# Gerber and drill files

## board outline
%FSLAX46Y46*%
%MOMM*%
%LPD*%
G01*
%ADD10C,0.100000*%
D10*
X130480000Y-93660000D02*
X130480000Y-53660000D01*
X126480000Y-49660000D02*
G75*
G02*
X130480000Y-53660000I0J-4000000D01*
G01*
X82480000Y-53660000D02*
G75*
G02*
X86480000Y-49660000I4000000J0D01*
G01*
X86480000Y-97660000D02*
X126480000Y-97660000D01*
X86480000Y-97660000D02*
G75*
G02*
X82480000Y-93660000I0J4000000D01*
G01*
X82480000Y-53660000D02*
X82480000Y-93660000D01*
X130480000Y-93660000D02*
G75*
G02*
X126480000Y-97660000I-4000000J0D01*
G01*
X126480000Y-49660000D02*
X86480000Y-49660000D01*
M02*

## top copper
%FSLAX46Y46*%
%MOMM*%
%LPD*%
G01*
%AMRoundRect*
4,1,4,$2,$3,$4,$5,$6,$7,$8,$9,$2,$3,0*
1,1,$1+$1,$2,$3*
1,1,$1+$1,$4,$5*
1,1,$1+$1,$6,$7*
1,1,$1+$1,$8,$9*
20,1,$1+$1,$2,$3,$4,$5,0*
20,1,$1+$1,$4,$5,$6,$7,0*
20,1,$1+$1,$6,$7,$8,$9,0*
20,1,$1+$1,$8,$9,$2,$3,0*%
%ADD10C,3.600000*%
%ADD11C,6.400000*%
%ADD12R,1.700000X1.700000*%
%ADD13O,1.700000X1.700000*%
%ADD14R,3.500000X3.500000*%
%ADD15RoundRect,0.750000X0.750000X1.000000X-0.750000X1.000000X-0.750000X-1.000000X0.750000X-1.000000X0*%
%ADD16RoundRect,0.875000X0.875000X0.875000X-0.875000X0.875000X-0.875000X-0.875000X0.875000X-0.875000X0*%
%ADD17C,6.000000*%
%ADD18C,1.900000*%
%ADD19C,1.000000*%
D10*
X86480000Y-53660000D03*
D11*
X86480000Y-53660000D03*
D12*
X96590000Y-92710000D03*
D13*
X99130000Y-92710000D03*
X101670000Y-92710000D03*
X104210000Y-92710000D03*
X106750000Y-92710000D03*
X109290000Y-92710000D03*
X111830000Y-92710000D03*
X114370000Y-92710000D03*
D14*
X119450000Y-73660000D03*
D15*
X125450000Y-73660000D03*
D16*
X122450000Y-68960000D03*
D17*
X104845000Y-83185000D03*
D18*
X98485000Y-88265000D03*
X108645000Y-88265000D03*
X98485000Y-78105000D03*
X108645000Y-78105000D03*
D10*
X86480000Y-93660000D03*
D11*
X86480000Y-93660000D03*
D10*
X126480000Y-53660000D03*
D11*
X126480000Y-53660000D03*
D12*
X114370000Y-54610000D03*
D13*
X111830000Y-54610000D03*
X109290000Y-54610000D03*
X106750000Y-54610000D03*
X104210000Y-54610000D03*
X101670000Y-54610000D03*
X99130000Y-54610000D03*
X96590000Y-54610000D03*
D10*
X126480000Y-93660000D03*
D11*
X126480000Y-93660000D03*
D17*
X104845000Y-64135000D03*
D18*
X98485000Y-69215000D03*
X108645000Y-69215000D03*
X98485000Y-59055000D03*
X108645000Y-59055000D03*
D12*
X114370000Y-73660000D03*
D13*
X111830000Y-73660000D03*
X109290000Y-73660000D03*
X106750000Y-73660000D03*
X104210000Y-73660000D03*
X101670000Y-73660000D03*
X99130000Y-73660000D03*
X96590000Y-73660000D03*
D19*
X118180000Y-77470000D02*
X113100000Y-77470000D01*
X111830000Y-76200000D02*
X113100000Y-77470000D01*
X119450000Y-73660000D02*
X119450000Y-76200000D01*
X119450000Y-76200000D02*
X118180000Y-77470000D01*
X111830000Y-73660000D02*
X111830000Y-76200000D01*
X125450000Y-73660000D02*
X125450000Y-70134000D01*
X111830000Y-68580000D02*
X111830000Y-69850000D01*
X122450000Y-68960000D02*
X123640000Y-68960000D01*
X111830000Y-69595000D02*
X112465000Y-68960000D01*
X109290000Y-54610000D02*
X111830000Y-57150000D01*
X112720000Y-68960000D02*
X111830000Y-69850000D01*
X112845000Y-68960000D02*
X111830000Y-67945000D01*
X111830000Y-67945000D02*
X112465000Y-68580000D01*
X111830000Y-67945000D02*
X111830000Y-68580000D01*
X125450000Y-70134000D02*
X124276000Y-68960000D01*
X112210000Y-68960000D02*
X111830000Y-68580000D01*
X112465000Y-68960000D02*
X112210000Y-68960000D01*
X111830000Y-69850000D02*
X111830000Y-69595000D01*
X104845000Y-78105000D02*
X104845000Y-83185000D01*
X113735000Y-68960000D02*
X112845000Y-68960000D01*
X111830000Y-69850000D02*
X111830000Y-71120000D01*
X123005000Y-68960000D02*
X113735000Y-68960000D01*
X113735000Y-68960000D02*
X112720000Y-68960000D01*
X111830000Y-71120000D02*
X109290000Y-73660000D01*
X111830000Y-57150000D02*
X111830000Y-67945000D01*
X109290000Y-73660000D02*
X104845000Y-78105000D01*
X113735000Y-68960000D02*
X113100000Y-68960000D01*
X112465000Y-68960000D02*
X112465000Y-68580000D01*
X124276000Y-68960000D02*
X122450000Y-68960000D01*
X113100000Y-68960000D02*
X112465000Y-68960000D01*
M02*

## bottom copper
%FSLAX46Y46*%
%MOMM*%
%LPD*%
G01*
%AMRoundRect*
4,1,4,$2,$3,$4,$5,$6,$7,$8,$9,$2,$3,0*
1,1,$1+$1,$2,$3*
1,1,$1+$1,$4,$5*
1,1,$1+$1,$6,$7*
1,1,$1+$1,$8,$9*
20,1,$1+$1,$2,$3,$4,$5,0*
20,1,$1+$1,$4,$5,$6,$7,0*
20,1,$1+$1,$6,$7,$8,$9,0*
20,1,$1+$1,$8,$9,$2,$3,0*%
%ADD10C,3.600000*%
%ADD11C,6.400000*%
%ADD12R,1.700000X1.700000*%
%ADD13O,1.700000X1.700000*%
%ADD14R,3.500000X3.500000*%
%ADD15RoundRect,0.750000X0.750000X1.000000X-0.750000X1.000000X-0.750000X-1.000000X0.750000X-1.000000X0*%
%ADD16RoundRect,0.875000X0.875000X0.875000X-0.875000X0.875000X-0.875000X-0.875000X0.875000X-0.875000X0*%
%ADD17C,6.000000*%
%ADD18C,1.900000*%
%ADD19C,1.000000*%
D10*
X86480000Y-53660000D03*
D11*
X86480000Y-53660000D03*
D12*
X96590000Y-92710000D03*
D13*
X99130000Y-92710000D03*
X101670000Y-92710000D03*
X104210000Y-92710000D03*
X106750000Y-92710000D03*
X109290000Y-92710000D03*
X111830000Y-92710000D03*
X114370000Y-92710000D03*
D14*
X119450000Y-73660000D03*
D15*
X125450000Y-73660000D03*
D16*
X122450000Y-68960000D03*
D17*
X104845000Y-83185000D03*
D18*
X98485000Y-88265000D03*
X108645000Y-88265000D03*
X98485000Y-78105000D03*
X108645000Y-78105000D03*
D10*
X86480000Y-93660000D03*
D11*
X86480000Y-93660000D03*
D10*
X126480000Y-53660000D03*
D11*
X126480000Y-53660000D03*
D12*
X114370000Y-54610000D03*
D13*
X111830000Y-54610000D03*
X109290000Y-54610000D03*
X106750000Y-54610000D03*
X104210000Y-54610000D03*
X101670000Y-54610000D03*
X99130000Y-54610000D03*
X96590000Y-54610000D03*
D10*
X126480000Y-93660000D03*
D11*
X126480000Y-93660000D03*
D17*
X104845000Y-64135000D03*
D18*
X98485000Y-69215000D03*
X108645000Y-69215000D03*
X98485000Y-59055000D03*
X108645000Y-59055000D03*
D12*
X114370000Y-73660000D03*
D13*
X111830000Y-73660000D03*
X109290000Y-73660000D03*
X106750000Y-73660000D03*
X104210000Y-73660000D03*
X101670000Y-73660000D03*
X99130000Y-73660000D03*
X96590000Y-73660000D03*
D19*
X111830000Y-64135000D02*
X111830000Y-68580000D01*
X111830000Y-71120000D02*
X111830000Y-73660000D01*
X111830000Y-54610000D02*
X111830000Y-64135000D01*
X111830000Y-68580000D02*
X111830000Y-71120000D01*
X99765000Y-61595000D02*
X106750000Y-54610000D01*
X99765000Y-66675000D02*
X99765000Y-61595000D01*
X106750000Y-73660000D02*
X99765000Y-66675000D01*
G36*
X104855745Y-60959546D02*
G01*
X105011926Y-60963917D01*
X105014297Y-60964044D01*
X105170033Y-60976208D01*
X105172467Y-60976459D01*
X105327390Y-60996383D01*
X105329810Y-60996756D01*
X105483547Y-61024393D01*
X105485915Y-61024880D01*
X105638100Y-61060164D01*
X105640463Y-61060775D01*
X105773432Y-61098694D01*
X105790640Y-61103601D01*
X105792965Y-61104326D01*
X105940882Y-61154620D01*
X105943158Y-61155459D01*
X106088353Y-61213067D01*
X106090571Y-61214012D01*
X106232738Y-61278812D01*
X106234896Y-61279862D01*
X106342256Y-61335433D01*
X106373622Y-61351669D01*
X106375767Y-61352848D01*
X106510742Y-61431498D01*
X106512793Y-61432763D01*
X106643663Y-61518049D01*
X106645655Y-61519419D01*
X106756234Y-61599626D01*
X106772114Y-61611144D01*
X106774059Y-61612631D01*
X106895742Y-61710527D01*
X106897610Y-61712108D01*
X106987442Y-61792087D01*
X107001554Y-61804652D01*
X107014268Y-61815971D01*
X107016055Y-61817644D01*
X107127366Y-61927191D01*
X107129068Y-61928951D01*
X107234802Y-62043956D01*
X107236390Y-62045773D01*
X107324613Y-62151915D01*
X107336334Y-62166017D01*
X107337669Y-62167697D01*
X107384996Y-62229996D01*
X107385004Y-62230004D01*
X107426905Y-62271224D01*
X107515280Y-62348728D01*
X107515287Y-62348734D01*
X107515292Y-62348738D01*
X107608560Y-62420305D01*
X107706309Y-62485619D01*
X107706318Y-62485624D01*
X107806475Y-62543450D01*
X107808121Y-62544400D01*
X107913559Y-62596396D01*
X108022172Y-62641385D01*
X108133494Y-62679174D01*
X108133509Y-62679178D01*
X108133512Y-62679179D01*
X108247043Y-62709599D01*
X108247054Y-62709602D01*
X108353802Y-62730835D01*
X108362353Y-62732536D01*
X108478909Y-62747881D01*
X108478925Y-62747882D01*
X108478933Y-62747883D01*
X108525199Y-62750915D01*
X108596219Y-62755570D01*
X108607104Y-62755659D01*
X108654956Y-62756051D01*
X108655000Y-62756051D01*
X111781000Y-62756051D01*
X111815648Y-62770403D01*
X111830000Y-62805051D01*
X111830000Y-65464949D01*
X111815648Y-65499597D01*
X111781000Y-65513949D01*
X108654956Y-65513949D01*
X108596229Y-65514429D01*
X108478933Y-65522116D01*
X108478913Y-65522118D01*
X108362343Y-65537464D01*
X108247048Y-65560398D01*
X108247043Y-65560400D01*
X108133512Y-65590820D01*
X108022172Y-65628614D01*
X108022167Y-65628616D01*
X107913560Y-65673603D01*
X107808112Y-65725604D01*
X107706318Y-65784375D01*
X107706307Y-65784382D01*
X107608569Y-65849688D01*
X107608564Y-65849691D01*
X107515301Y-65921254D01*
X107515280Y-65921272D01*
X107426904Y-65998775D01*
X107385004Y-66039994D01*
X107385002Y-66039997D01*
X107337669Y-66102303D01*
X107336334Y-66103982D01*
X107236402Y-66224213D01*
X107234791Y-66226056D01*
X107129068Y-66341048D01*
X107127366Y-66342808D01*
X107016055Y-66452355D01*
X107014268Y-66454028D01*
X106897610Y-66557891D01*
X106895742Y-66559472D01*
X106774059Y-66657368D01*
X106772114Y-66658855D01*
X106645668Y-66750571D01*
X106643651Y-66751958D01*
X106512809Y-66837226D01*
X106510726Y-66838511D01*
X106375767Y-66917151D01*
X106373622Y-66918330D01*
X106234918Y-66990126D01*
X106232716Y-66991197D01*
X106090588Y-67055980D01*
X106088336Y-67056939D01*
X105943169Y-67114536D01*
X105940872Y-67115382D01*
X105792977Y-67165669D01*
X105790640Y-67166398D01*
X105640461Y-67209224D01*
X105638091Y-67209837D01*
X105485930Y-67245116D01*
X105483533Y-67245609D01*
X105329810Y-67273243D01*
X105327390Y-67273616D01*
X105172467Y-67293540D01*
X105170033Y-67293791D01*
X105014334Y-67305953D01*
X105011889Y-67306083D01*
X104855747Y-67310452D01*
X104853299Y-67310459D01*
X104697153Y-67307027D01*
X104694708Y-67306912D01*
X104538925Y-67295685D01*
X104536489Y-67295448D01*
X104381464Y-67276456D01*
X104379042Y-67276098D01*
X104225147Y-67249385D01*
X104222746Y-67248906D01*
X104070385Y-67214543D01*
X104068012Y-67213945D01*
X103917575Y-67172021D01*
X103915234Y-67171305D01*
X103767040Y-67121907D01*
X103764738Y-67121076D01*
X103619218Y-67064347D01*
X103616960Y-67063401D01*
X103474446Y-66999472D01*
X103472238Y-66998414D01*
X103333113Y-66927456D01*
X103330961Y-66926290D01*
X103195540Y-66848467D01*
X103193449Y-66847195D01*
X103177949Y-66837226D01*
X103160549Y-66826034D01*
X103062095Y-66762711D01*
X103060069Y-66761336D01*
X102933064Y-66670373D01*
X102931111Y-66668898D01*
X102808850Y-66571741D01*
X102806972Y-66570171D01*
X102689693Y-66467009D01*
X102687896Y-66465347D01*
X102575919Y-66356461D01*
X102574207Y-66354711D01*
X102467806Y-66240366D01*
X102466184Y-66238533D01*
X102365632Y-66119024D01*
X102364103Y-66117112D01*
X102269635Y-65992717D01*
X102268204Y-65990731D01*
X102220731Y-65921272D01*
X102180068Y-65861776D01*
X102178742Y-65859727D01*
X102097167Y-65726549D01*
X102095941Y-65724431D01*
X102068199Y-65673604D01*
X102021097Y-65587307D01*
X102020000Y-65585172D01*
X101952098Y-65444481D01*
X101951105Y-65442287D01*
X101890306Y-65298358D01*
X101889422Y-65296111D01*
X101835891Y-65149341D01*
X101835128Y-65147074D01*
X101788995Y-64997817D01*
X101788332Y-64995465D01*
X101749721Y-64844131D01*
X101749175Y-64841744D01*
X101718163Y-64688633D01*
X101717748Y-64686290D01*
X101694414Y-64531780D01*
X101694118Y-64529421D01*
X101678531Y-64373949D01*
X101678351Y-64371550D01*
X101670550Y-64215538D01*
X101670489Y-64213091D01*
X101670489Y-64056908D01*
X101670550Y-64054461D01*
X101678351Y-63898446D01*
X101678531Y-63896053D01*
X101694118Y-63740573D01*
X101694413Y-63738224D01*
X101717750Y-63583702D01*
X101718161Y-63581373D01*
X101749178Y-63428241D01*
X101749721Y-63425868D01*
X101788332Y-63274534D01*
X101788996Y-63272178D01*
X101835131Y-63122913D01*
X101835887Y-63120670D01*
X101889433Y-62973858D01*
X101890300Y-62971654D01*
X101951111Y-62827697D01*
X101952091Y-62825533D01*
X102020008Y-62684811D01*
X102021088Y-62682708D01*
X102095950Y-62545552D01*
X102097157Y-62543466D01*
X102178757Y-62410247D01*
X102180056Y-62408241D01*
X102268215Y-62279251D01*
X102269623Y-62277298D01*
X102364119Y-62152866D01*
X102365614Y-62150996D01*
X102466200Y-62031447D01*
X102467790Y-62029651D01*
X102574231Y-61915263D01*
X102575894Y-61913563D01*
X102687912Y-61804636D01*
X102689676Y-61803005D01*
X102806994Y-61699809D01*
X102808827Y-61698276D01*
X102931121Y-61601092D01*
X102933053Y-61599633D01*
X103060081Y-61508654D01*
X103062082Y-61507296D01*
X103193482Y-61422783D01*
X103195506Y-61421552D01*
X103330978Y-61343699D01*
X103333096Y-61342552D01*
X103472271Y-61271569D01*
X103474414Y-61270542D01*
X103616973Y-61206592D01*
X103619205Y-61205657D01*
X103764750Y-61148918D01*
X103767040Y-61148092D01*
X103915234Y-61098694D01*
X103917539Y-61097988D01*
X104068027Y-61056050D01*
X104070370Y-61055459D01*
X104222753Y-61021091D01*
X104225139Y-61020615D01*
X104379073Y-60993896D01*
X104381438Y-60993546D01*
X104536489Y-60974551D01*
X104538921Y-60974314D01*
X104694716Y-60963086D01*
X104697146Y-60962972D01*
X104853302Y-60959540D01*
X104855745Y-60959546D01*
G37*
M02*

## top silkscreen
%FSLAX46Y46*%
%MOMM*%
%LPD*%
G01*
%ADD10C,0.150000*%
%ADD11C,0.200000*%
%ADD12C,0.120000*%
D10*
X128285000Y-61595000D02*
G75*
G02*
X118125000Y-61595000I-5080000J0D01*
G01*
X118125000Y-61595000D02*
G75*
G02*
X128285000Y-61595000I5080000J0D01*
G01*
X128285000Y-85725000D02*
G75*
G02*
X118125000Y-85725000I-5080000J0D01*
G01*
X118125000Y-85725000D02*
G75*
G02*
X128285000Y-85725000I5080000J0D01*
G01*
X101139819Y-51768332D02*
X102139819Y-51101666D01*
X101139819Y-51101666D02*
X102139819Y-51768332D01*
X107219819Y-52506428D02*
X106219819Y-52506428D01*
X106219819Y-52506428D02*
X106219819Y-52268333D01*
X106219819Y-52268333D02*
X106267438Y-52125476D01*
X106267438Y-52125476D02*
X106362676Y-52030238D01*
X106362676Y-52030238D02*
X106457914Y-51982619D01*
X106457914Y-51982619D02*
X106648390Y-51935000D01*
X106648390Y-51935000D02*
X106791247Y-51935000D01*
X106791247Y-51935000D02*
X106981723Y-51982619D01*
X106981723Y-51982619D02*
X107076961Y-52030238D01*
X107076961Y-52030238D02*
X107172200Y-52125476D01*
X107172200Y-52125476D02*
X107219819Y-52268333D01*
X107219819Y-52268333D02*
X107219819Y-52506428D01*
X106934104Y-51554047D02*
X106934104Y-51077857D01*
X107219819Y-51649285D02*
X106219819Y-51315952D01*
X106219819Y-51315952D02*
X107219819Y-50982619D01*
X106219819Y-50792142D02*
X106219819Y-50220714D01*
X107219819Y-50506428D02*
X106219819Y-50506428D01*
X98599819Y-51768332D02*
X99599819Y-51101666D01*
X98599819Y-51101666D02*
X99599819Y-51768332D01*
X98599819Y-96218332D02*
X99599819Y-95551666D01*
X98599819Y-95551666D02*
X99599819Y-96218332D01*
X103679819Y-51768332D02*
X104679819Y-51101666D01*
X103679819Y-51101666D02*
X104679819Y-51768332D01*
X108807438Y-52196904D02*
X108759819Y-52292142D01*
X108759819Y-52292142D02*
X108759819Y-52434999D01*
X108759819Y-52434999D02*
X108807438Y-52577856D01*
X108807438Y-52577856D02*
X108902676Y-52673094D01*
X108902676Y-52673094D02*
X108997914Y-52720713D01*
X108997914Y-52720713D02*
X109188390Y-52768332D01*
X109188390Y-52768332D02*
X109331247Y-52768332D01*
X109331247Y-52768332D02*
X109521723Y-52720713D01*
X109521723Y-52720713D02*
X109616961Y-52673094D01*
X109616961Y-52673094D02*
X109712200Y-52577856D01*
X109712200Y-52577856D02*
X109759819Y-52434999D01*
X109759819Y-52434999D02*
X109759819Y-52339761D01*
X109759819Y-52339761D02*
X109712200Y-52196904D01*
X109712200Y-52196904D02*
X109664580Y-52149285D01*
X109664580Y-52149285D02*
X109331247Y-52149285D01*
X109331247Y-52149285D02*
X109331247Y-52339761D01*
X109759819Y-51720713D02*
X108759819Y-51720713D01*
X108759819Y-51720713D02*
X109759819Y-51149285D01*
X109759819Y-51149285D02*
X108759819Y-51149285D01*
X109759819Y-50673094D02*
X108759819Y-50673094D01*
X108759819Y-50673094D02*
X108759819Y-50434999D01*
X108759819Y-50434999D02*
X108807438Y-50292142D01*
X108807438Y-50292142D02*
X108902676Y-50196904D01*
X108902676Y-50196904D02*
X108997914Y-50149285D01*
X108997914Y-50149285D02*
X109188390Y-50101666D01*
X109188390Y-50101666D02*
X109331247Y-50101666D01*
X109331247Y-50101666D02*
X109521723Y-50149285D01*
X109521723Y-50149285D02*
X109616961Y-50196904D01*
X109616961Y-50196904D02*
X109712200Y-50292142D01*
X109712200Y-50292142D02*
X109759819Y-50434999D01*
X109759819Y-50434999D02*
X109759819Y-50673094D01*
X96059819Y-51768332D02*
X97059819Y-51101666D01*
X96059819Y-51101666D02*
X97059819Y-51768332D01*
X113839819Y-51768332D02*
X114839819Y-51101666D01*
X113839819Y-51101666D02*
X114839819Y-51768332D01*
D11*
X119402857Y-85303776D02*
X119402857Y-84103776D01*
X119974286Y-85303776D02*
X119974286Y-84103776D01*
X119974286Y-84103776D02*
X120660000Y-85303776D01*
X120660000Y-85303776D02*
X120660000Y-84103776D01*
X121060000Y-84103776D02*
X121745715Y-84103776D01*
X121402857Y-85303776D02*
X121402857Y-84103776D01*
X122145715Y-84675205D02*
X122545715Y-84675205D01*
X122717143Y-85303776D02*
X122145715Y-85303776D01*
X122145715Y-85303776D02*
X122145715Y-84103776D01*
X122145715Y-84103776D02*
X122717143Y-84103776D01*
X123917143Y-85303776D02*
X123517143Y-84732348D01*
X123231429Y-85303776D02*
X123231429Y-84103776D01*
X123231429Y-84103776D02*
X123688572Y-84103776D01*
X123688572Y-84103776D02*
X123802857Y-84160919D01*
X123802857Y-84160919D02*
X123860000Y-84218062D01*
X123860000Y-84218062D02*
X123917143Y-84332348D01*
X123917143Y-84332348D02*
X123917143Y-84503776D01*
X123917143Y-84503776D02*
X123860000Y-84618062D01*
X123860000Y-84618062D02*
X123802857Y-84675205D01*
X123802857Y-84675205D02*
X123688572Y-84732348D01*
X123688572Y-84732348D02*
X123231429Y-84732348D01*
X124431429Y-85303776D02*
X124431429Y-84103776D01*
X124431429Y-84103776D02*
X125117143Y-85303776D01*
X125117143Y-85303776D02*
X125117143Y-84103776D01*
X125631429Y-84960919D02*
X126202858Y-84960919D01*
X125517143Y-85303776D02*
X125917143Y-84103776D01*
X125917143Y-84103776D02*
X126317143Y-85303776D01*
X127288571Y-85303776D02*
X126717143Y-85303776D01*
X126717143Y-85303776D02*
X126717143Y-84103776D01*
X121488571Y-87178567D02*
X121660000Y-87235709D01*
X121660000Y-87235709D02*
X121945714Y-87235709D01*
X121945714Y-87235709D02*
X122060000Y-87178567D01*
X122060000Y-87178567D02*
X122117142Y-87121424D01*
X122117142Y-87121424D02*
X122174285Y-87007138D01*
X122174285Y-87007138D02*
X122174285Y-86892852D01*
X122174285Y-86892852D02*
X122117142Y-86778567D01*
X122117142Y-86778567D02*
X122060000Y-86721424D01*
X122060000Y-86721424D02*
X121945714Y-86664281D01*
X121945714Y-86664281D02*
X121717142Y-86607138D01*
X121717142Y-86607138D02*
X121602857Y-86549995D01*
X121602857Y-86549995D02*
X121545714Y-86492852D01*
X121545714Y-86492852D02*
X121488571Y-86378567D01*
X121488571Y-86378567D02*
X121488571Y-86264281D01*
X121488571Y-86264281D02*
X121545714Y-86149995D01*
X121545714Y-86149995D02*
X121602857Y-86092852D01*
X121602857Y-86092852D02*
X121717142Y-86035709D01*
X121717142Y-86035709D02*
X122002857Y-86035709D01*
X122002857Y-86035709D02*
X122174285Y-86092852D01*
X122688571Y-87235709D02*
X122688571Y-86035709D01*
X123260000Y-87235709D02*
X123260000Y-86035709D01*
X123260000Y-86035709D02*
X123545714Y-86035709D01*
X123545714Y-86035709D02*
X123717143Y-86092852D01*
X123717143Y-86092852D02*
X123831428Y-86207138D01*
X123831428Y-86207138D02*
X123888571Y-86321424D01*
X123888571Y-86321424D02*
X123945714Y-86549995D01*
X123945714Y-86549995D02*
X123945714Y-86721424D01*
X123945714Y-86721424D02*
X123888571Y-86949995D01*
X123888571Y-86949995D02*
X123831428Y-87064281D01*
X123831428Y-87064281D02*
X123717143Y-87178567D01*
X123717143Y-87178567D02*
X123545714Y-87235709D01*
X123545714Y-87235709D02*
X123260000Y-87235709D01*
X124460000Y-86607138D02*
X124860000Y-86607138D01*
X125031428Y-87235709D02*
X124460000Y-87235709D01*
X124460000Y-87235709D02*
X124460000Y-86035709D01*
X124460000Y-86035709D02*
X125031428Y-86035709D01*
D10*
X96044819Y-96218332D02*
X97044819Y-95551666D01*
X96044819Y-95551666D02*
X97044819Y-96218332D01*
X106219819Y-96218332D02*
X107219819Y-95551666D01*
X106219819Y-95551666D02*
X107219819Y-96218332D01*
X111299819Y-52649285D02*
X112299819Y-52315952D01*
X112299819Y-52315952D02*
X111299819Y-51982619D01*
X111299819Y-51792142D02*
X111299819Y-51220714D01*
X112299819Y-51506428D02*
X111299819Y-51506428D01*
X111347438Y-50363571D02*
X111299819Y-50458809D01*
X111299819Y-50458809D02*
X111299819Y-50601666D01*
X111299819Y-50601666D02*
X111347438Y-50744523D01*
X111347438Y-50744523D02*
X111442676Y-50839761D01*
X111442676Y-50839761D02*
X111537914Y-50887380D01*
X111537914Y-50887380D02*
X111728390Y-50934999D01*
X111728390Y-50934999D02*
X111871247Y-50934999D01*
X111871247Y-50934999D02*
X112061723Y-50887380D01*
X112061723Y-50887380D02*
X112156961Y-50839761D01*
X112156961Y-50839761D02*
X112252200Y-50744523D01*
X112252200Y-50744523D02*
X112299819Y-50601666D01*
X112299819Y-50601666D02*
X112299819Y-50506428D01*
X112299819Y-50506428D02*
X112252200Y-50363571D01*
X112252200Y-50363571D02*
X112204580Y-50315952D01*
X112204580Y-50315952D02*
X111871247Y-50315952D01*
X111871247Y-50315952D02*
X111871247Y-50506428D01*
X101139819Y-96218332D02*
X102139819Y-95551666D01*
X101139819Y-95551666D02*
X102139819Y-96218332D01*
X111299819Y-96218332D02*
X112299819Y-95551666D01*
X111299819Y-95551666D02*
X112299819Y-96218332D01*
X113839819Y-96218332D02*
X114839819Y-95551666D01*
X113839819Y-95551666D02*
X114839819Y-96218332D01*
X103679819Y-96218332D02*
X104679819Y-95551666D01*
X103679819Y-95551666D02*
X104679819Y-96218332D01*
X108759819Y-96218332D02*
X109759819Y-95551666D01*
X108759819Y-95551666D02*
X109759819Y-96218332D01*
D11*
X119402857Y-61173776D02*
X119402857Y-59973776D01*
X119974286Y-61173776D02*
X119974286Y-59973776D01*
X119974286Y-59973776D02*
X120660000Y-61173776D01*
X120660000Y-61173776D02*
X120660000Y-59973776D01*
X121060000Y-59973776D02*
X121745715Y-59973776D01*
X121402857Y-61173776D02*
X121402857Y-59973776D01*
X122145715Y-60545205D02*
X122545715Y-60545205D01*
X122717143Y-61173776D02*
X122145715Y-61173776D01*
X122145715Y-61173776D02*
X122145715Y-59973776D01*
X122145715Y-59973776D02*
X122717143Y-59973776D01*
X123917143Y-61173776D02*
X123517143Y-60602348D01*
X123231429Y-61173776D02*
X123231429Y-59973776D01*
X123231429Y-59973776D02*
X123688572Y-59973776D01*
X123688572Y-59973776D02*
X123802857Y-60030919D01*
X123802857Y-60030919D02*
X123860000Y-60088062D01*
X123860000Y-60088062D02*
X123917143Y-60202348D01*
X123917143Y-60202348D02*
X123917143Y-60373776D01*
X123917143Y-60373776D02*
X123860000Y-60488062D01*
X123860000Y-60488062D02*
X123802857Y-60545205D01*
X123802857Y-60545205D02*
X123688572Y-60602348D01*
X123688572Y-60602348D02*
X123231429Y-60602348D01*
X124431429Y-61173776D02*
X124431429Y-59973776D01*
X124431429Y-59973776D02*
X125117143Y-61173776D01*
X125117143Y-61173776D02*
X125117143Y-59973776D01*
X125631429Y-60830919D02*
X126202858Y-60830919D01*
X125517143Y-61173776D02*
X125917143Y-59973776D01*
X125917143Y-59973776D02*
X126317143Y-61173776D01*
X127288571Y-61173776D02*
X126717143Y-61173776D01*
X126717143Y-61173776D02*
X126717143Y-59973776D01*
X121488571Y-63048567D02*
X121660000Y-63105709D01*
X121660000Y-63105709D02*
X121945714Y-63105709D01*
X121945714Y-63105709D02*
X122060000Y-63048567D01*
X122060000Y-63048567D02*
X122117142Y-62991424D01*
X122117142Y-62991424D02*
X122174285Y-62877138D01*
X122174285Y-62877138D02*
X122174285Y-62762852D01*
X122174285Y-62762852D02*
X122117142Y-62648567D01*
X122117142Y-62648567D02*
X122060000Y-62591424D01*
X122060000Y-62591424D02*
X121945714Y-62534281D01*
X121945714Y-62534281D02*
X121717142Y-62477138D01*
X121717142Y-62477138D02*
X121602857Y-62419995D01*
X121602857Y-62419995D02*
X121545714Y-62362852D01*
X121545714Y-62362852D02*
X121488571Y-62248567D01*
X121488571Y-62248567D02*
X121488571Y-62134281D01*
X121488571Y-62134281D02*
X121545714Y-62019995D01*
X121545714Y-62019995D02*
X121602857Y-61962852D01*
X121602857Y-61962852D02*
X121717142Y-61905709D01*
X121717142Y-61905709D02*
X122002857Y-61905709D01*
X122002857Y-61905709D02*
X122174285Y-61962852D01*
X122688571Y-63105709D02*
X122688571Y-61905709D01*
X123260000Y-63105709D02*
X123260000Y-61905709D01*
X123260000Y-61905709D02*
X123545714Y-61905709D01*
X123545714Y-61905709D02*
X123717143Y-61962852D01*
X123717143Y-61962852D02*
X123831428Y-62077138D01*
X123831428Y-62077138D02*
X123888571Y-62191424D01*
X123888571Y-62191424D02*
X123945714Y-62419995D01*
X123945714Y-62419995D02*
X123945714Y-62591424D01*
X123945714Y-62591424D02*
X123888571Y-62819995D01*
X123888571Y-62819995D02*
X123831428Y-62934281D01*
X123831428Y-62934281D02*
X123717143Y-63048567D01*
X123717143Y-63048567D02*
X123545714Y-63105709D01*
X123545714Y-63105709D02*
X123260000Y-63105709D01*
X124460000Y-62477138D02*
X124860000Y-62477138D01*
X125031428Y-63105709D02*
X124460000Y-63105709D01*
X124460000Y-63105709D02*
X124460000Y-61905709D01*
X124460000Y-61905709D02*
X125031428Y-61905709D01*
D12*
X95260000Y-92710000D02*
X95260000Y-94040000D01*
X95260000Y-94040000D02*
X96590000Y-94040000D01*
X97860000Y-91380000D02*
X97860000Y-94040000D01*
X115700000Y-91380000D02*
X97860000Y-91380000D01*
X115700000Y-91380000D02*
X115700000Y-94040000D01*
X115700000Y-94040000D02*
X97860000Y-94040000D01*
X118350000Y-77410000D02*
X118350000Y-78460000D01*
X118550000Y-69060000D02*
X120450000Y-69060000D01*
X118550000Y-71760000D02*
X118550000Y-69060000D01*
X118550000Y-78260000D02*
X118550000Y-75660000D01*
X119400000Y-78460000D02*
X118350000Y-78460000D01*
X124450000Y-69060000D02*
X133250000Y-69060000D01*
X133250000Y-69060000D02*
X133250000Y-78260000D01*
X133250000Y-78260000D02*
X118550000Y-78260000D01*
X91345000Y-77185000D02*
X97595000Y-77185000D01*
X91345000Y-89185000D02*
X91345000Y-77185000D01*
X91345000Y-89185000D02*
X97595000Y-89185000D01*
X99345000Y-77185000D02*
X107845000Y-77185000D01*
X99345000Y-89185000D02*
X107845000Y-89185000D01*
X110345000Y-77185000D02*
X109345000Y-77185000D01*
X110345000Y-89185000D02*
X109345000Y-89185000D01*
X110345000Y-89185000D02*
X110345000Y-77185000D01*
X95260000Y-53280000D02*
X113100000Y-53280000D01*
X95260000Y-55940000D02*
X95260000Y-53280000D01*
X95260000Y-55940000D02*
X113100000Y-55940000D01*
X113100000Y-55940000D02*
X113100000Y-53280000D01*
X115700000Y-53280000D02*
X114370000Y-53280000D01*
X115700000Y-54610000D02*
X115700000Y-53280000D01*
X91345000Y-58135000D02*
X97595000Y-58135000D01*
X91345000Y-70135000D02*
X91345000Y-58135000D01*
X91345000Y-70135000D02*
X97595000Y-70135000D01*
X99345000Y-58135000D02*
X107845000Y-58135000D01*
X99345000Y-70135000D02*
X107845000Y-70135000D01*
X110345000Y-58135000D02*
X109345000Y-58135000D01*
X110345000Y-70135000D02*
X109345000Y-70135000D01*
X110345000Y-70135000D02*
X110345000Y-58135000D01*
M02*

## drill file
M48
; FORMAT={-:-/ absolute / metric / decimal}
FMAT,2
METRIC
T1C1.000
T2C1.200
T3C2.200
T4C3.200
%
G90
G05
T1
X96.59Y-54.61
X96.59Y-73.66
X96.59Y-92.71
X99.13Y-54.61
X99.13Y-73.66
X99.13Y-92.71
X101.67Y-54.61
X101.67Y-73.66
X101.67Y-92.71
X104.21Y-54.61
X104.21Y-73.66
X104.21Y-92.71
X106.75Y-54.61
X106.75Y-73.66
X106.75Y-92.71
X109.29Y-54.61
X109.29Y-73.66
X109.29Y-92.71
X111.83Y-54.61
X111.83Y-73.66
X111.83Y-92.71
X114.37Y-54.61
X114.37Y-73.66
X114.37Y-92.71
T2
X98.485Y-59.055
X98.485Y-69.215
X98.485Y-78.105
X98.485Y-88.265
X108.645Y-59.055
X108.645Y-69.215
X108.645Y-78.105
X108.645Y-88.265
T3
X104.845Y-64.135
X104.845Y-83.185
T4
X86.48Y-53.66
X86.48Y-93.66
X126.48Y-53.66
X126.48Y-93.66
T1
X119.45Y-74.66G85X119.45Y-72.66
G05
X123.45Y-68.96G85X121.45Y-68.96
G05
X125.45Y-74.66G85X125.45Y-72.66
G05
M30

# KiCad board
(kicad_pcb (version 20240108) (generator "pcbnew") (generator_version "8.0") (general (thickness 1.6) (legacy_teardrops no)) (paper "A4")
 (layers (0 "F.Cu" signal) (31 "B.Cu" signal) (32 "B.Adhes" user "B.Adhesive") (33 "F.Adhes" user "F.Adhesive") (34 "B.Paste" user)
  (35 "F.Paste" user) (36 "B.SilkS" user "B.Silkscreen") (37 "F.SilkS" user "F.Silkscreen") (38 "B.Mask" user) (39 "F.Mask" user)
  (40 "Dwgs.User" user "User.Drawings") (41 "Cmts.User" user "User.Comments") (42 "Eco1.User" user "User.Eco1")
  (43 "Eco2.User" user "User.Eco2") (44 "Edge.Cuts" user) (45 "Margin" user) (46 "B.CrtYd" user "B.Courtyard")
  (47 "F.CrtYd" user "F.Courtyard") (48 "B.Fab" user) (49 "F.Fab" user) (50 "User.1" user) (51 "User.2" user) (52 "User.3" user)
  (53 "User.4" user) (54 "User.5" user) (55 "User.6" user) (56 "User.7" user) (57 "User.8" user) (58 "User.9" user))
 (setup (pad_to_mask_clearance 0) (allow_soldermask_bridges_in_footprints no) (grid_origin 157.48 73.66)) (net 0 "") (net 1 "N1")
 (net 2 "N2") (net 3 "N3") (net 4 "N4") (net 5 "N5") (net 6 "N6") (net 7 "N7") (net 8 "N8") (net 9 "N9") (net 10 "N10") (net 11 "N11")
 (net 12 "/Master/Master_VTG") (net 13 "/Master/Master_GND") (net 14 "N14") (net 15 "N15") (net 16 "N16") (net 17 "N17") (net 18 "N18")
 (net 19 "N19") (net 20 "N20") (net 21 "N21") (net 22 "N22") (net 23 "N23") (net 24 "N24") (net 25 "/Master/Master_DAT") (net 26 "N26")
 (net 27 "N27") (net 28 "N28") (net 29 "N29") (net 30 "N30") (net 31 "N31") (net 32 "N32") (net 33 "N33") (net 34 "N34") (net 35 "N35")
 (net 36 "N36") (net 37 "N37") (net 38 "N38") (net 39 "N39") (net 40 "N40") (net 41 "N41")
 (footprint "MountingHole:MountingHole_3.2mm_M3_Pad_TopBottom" (layer "F.Cu") (at 86.48 53.66)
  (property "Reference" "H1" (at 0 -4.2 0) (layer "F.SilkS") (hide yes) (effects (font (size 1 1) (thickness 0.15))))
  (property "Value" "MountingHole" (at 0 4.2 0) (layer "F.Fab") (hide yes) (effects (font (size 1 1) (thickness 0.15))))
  (pad "1" thru_hole circle (at 0 0) (size 3.6 3.6) (drill 3.2) (layers "*.Cu" "*.Mask") (remove_unused_layers no) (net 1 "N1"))
  (pad "1" connect circle (at 0 0) (size 6.4 6.4) (layers "F.Cu" "F.Mask") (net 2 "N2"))
  (pad "1" connect circle (at 0 0) (size 6.4 6.4) (layers "B.Cu" "B.Mask") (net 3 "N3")))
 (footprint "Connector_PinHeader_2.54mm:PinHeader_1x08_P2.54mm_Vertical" (layer "F.Cu") (at 96.59 92.71 90)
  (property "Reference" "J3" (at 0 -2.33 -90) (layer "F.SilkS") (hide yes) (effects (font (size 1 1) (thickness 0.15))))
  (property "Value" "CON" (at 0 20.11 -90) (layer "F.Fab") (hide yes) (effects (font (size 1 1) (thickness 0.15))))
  (fp_line (start 0 -1.33) (end -1.33 -1.33) (stroke (width 0.12) (type solid)) (layer "F.SilkS"))
  (fp_line (start -1.33 -1.33) (end -1.33 0) (stroke (width 0.12) (type solid)) (layer "F.SilkS"))
  (fp_line (start 1.33 1.27) (end -1.33 1.27) (stroke (width 0.12) (type solid)) (layer "F.SilkS"))
  (fp_line (start 1.33 19.11) (end 1.33 1.27) (stroke (width 0.12) (type solid)) (layer "F.SilkS"))
  (fp_line (start 1.33 19.11) (end -1.33 19.11) (stroke (width 0.12) (type solid)) (layer "F.SilkS"))
  (fp_line (start -1.33 19.11) (end -1.33 1.27) (stroke (width 0.12) (type solid)) (layer "F.SilkS"))
  (pad "1" thru_hole rect (at 0 0 90) (size 1.7 1.7) (drill 1) (layers "*.Cu" "*.Mask") (remove_unused_layers no) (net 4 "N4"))
  (pad "2" thru_hole oval (at 0 2.54 90) (size 1.7 1.7) (drill 1) (layers "*.Cu" "*.Mask") (remove_unused_layers no) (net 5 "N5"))
  (pad "3" thru_hole oval (at 0 5.08 90) (size 1.7 1.7) (drill 1) (layers "*.Cu" "*.Mask") (remove_unused_layers no) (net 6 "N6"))
  (pad "4" thru_hole oval (at 0 7.62 90) (size 1.7 1.7) (drill 1) (layers "*.Cu" "*.Mask") (remove_unused_layers no) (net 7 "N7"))
  (pad "5" thru_hole oval (at 0 10.16 90) (size 1.7 1.7) (drill 1) (layers "*.Cu" "*.Mask") (remove_unused_layers no) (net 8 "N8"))
  (pad "6" thru_hole oval (at 0 12.7 90) (size 1.7 1.7) (drill 1) (layers "*.Cu" "*.Mask") (remove_unused_layers no) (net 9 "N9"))
  (pad "7" thru_hole oval (at 0 15.24 90) (size 1.7 1.7) (drill 1) (layers "*.Cu" "*.Mask") (remove_unused_layers no) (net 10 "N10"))
  (pad "8" thru_hole oval (at 0 17.78 90) (size 1.7 1.7) (drill 1) (layers "*.Cu" "*.Mask") (remove_unused_layers no) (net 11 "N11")))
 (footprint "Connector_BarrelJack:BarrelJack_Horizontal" (layer "F.Cu") (at 119.45 73.66 180)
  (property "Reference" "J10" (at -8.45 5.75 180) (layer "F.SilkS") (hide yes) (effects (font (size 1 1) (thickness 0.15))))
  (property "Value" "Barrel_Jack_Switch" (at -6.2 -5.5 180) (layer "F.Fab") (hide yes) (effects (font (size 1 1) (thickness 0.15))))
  (fp_line (start 1.1 -3.75) (end 1.1 -4.8) (stroke (width 0.12) (type solid)) (layer "F.SilkS"))
  (fp_line (start 0.9 4.6) (end -1 4.6) (stroke (width 0.12) (type solid)) (layer "F.SilkS"))
  (fp_line (start 0.9 1.9) (end 0.9 4.6) (stroke (width 0.12) (type solid)) (layer "F.SilkS"))
  (fp_line (start 0.9 -4.6) (end 0.9 -2) (stroke (width 0.12) (type solid)) (layer "F.SilkS"))
  (fp_line (start 0.05 -4.8) (end 1.1 -4.8) (stroke (width 0.12) (type solid)) (layer "F.SilkS"))
  (fp_line (start -5 4.6) (end -13.8 4.6) (stroke (width 0.12) (type solid)) (layer "F.SilkS"))
  (fp_line (start -13.8 4.6) (end -13.8 -4.6) (stroke (width 0.12) (type solid)) (layer "F.SilkS"))
  (fp_line (start -13.8 -4.6) (end 0.9 -4.6) (stroke (width 0.12) (type solid)) (layer "F.SilkS"))
  (pad "1" thru_hole rect (at 0 0 180) (size 3.5 3.5) (drill oval 1 3) (layers "*.Cu" "*.Mask") (remove_unused_layers no)
   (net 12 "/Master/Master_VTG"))
  (pad "2" thru_hole roundrect (at -6 0 180) (size 3 3.5) (drill oval 1 3) (layers "*.Cu" "*.Mask") (remove_unused_layers no)
   (roundrect_rratio 0.25) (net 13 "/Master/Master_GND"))
  (pad "3" thru_hole roundrect (at -3 4.7 180) (size 3.5 3.5) (drill oval 3 1) (layers "*.Cu" "*.Mask") (remove_unused_layers no)
   (roundrect_rratio 0.25) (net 13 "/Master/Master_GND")))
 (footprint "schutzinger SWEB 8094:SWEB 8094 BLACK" (layer "F.Cu") (at 104.845 83.185 90)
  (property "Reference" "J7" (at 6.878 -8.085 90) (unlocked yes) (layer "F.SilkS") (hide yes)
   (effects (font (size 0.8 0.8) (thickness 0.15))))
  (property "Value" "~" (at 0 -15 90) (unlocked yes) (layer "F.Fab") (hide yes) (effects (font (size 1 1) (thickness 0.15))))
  (fp_line (start 6 -13.5) (end 6 -7.25) (stroke (width 0.12) (type solid)) (layer "F.SilkS"))
  (fp_line (start -6 -13.5) (end 6 -13.5) (stroke (width 0.12) (type solid)) (layer "F.SilkS"))
  (fp_line (start -6 -13.5) (end -6 -7.25) (stroke (width 0.12) (type solid)) (layer "F.SilkS"))
  (fp_line (start 6 -5.5) (end 6 3) (stroke (width 0.12) (type solid)) (layer "F.SilkS"))
  (fp_line (start -6 -5.5) (end -6 3) (stroke (width 0.12) (type solid)) (layer "F.SilkS"))
  (fp_line (start 6 5.5) (end 6 4.5) (stroke (width 0.12) (type solid)) (layer "F.SilkS"))
  (fp_line (start -6 5.5) (end -6 4.5) (stroke (width 0.12) (type solid)) (layer "F.SilkS"))
  (fp_line (start -6 5.5) (end 6 5.5) (stroke (width 0.12) (type solid)) (layer "F.SilkS"))
  (pad "1" thru_hole circle (at 0 0 90) (size 6 6) (drill 2.2) (layers "*.Cu" "*.Mask") (remove_unused_layers no)
   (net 13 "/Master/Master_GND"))
  (pad "MP" thru_hole circle (at -5.08 -6.36 90) (size 1.9 1.9) (drill 1.2) (layers "*.Cu" "*.Mask") (remove_unused_layers no)
   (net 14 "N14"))
  (pad "MP" thru_hole circle (at -5.08 3.8 90) (size 1.9 1.9) (drill 1.2) (layers "*.Cu" "*.Mask") (remove_unused_layers no) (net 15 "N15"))
  (pad "MP" thru_hole circle (at 5.08 -6.36 90) (size 1.9 1.9) (drill 1.2) (layers "*.Cu" "*.Mask") (remove_unused_layers no) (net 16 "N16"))
  (pad "MP" thru_hole circle (at 5.08 3.8 90) (size 1.9 1.9) (drill 1.2) (layers "*.Cu" "*.Mask") (remove_unused_layers no) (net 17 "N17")))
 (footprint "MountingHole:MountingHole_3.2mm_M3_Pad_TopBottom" (layer "F.Cu") (at 86.48 93.66)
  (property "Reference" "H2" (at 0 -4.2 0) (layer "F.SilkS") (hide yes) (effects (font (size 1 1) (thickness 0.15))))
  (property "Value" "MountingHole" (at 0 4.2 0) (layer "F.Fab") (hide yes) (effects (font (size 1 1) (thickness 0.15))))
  (pad "1" thru_hole circle (at 0 0) (size 3.6 3.6) (drill 3.2) (layers "*.Cu" "*.Mask") (remove_unused_layers no) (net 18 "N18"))
  (pad "1" connect circle (at 0 0) (size 6.4 6.4) (layers "F.Cu" "F.Mask") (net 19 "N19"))
  (pad "1" connect circle (at 0 0) (size 6.4 6.4) (layers "B.Cu" "B.Mask") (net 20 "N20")))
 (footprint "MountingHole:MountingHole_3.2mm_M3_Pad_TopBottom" (layer "F.Cu") (at 126.48 53.66)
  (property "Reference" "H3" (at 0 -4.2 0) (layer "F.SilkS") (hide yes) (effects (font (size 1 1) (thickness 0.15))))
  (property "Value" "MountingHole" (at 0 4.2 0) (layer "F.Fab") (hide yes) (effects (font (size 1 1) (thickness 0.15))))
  (pad "1" thru_hole circle (at 0 0) (size 3.6 3.6) (drill 3.2) (layers "*.Cu" "*.Mask") (remove_unused_layers no) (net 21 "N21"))
  (pad "1" connect circle (at 0 0) (size 6.4 6.4) (layers "F.Cu" "F.Mask") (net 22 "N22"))
  (pad "1" connect circle (at 0 0) (size 6.4 6.4) (layers "B.Cu" "B.Mask") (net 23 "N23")))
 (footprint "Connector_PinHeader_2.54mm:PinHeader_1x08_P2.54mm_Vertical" (layer "F.Cu") (at 114.37 54.61 -90)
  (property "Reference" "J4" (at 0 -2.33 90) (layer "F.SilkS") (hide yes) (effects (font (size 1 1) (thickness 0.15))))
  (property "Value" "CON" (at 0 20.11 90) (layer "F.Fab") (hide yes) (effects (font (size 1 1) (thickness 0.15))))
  (fp_line (start -1.33 19.11) (end -1.33 1.27) (stroke (width 0.12) (type solid)) (layer "F.SilkS"))
  (fp_line (start 1.33 19.11) (end -1.33 19.11) (stroke (width 0.12) (type solid)) (layer "F.SilkS"))
  (fp_line (start 1.33 19.11) (end 1.33 1.27) (stroke (width 0.12) (type solid)) (layer "F.SilkS"))
  (fp_line (start 1.33 1.27) (end -1.33 1.27) (stroke (width 0.12) (type solid)) (layer "F.SilkS"))
  (fp_line (start -1.33 -1.33) (end -1.33 0) (stroke (width 0.12) (type solid)) (layer "F.SilkS"))
  (fp_line (start 0 -1.33) (end -1.33 -1.33) (stroke (width 0.12) (type solid)) (layer "F.SilkS"))
  (pad "1" thru_hole rect (at 0 0 270) (size 1.7 1.7) (drill 1) (layers "*.Cu" "*.Mask") (remove_unused_layers no) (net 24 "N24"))
  (pad "2" thru_hole oval (at 0 2.54 270) (size 1.7 1.7) (drill 1) (layers "*.Cu" "*.Mask") (remove_unused_layers no)
   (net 12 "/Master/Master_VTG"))
  (pad "3" thru_hole oval (at 0 5.08 270) (size 1.7 1.7) (drill 1) (layers "*.Cu" "*.Mask") (remove_unused_layers no)
   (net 13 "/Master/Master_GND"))
  (pad "4" thru_hole oval (at 0 7.62 270) (size 1.7 1.7) (drill 1) (layers "*.Cu" "*.Mask") (remove_unused_layers no)
   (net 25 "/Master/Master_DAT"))
  (pad "5" thru_hole oval (at 0 10.16 270) (size 1.7 1.7) (drill 1) (layers "*.Cu" "*.Mask") (remove_unused_layers no) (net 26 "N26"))
  (pad "6" thru_hole oval (at 0 12.7 270) (size 1.7 1.7) (drill 1) (layers "*.Cu" "*.Mask") (remove_unused_layers no) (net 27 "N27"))
  (pad "7" thru_hole oval (at 0 15.24 270) (size 1.7 1.7) (drill 1) (layers "*.Cu" "*.Mask") (remove_unused_layers no) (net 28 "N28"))
  (pad "8" thru_hole oval (at 0 17.78 270) (size 1.7 1.7) (drill 1) (layers "*.Cu" "*.Mask") (remove_unused_layers no) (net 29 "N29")))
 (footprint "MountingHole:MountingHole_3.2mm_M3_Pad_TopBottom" (layer "F.Cu") (at 126.48 93.66)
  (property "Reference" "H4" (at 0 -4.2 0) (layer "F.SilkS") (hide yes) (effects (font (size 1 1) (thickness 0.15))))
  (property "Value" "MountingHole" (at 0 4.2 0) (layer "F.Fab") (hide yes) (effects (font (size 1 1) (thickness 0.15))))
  (pad "1" thru_hole circle (at 0 0) (size 3.6 3.6) (drill 3.2) (layers "*.Cu" "*.Mask") (remove_unused_layers no) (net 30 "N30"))
  (pad "1" connect circle (at 0 0) (size 6.4 6.4) (layers "F.Cu" "F.Mask") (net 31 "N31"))
  (pad "1" connect circle (at 0 0) (size 6.4 6.4) (layers "B.Cu" "B.Mask") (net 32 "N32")))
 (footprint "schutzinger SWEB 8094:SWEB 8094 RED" (layer "F.Cu") (at 104.845 64.135 90)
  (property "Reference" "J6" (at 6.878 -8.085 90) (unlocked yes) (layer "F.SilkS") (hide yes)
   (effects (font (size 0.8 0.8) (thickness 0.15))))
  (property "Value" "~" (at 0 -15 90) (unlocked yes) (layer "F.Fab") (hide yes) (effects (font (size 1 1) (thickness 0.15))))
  (fp_line (start 6 -13.5) (end 6 -7.25) (stroke (width 0.12) (type solid)) (layer "F.SilkS"))
  (fp_line (start -6 -13.5) (end 6 -13.5) (stroke (width 0.12) (type solid)) (layer "F.SilkS"))
  (fp_line (start -6 -13.5) (end -6 -7.25) (stroke (width 0.12) (type solid)) (layer "F.SilkS"))
  (fp_line (start 6 -5.5) (end 6 3) (stroke (width 0.12) (type solid)) (layer "F.SilkS"))
  (fp_line (start -6 -5.5) (end -6 3) (stroke (width 0.12) (type solid)) (layer "F.SilkS"))
  (fp_line (start 6 5.5) (end 6 4.5) (stroke (width 0.12) (type solid)) (layer "F.SilkS"))
  (fp_line (start -6 5.5) (end -6 4.5) (stroke (width 0.12) (type solid)) (layer "F.SilkS"))
  (fp_line (start -6 5.5) (end 6 5.5) (stroke (width 0.12) (type solid)) (layer "F.SilkS"))
  (pad "1" thru_hole circle (at 0 0 90) (size 6 6) (drill 2.2) (layers "*.Cu" "*.Mask") (remove_unused_layers no)
   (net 12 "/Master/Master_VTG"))
  (pad "MP" thru_hole circle (at -5.08 -6.36 90) (size 1.9 1.9) (drill 1.2) (layers "*.Cu" "*.Mask") (remove_unused_layers no)
   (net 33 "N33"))
  (pad "MP" thru_hole circle (at -5.08 3.8 90) (size 1.9 1.9) (drill 1.2) (layers "*.Cu" "*.Mask") (remove_unused_layers no) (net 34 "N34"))
  (pad "MP" thru_hole circle (at 5.08 -6.36 90) (size 1.9 1.9) (drill 1.2) (layers "*.Cu" "*.Mask") (remove_unused_layers no) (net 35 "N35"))
  (pad "MP" thru_hole circle (at 5.08 3.8 90) (size 1.9 1.9) (drill 1.2) (layers "*.Cu" "*.Mask") (remove_unused_layers no) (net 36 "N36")))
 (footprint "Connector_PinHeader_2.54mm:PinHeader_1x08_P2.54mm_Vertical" (layer "B.Cu") (at 114.37 73.66 90)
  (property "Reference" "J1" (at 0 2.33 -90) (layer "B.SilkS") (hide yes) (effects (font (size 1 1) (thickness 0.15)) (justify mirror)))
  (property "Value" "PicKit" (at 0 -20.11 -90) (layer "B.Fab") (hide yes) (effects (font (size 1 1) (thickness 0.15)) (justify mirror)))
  (pad "1" thru_hole rect (at 0 0 90) (size 1.7 1.7) (drill 1) (layers "*.Cu" "*.Mask") (remove_unused_layers no) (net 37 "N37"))
  (pad "2" thru_hole oval (at 0 -2.54 90) (size 1.7 1.7) (drill 1) (layers "*.Cu" "*.Mask") (remove_unused_layers no)
   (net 12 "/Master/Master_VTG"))
  (pad "3" thru_hole oval (at 0 -5.08 90) (size 1.7 1.7) (drill 1) (layers "*.Cu" "*.Mask") (remove_unused_layers no)
   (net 13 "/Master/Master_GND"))
  (pad "4" thru_hole oval (at 0 -7.62 90) (size 1.7 1.7) (drill 1) (layers "*.Cu" "*.Mask") (remove_unused_layers no)
   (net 25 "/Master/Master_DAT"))
  (pad "5" thru_hole oval (at 0 -10.16 90) (size 1.7 1.7) (drill 1) (layers "*.Cu" "*.Mask") (remove_unused_layers no) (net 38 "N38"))
  (pad "6" thru_hole oval (at 0 -12.7 90) (size 1.7 1.7) (drill 1) (layers "*.Cu" "*.Mask") (remove_unused_layers no) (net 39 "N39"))
  (pad "7" thru_hole oval (at 0 -15.24 90) (size 1.7 1.7) (drill 1) (layers "*.Cu" "*.Mask") (remove_unused_layers no) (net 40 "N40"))
  (pad "8" thru_hole oval (at 0 -17.78 90) (size 1.7 1.7) (drill 1) (layers "*.Cu" "*.Mask") (remove_unused_layers no) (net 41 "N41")))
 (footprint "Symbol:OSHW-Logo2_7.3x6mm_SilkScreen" (layer "B.Cu") (at 86.43 63.5 90)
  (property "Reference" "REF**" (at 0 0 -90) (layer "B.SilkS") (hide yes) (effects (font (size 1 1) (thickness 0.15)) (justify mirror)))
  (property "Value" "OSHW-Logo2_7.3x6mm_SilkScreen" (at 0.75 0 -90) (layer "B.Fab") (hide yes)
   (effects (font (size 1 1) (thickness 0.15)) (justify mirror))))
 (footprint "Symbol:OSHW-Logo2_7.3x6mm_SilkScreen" (layer "B.Cu") (at 86.43 83.82 90)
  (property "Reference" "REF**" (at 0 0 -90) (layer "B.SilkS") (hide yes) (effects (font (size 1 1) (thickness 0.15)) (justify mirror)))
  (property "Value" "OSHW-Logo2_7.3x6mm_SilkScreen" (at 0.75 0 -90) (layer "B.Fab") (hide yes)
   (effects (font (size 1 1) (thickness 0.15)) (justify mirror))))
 (gr_circle (center 123.205 61.595) (end 118.125 61.595) (stroke (width 0.15) (type default)) (fill none) (layer "F.SilkS"))
 (gr_circle (center 123.205 85.725) (end 118.125 85.725) (stroke (width 0.15) (type default)) (fill none) (layer "F.SilkS"))
 (gr_line (start 130.48 93.66) (end 130.48 53.66) (stroke (width 0.1) (type default)) (layer "Edge.Cuts"))
 (gr_arc (start 126.48 49.66) (mid 129.308427 50.831573) (end 130.48 53.66) (stroke (width 0.1) (type default)) (layer "Edge.Cuts"))
 (gr_arc (start 82.48 53.66) (mid 83.651573 50.831573) (end 86.48 49.66) (stroke (width 0.1) (type default)) (layer "Edge.Cuts"))
 (gr_line (start 86.48 97.66) (end 126.48 97.66) (stroke (width 0.1) (type default)) (layer "Edge.Cuts"))
 (gr_arc (start 86.48 97.66) (mid 83.651573 96.488427) (end 82.48 93.66) (stroke (width 0.1) (type default)) (layer "Edge.Cuts"))
 (gr_line (start 82.48 53.66) (end 82.48 93.66) (stroke (width 0.1) (type default)) (layer "Edge.Cuts"))
 (gr_arc (start 130.48 93.66) (mid 129.308427 96.488427) (end 126.48 97.66) (stroke (width 0.1) (type default)) (layer "Edge.Cuts"))
 (gr_line (start 126.48 49.66) (end 86.48 49.66) (stroke (width 0.1) (type default)) (layer "Edge.Cuts"))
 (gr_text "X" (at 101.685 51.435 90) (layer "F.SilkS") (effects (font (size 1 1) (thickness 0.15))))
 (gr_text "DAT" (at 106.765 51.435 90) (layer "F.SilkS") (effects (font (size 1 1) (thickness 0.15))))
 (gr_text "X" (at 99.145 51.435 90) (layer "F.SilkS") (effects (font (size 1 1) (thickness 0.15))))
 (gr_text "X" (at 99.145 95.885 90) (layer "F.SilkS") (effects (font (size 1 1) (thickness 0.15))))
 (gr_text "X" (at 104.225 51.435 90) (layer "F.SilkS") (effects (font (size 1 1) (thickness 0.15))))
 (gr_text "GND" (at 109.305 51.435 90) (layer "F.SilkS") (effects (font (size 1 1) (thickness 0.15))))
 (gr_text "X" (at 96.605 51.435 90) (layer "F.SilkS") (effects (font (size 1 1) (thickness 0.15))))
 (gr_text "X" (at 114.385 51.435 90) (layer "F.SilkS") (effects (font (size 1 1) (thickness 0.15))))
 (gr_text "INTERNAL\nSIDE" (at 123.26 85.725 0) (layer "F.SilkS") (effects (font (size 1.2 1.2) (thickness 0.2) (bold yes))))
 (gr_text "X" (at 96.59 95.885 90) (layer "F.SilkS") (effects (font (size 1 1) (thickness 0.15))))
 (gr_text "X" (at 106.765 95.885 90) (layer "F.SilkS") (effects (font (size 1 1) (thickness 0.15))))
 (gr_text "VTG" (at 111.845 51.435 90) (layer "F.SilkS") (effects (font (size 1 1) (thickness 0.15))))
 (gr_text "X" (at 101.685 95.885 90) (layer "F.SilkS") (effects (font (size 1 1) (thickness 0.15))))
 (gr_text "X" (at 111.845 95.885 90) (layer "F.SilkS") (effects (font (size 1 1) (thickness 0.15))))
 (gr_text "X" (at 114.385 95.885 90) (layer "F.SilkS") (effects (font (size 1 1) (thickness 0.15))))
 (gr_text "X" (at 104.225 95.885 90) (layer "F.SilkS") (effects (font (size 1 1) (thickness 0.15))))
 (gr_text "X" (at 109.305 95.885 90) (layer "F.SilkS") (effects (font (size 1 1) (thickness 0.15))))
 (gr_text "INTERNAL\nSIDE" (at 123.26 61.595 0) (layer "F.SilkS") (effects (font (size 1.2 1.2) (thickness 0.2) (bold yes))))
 (segment (start 118.18 77.47) (end 113.1 77.47) (width 1) (layer "F.Cu") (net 12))
 (segment (start 111.83 76.2) (end 113.1 77.47) (width 1) (layer "F.Cu") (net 12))
 (segment (start 119.45 73.66) (end 119.45 76.2) (width 1) (layer "F.Cu") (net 12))
 (segment (start 119.45 76.2) (end 118.18 77.47) (width 1) (layer "F.Cu") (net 12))
 (segment (start 111.83 73.66) (end 111.83 76.2) (width 1) (layer "F.Cu") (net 12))
 (segment (start 111.83 64.135) (end 111.83 68.58) (width 1) (layer "B.Cu") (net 12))
 (segment (start 111.83 71.12) (end 111.83 73.66) (width 1) (layer "B.Cu") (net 12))
 (segment (start 111.83 54.61) (end 111.83 64.135) (width 1) (layer "B.Cu") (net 12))
 (segment (start 111.83 68.58) (end 111.83 71.12) (width 1) (layer "B.Cu") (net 12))
 (segment (start 99.765 61.595) (end 106.75 54.61) (width 1) (layer "B.Cu") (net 25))
 (segment (start 99.765 66.675) (end 99.765 61.595) (width 1) (layer "B.Cu") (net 25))
 (segment (start 106.75 73.66) (end 99.765 66.675) (width 1) (layer "B.Cu") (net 25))
 (segment (start 125.45 73.66) (end 125.45 70.134) (width 1) (layer "F.Cu") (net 13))
 (segment (start 111.83 68.58) (end 111.83 69.85) (width 1) (layer "F.Cu") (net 13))
 (segment (start 122.45 68.96) (end 123.64 68.96) (width 1) (layer "F.Cu") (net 13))
 (segment (start 111.83 69.595) (end 112.465 68.96) (width 1) (layer "F.Cu") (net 13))
 (segment (start 109.29 54.61) (end 111.83 57.15) (width 1) (layer "F.Cu") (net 13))
 (segment (start 112.72 68.96) (end 111.83 69.85) (width 1) (layer "F.Cu") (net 13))
 (segment (start 112.845 68.96) (end 111.83 67.945) (width 1) (layer "F.Cu") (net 13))
 (segment (start 111.83 67.945) (end 112.465 68.58) (width 1) (layer "F.Cu") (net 13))
 (segment (start 111.83 67.945) (end 111.83 68.58) (width 1) (layer "F.Cu") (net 13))
 (segment (start 125.45 70.134) (end 124.276 68.96) (width 1) (layer "F.Cu") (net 13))
 (segment (start 112.21 68.96) (end 111.83 68.58) (width 1) (layer "F.Cu") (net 13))
 (segment (start 112.465 68.96) (end 112.21 68.96) (width 1) (layer "F.Cu") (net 13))
 (segment (start 111.83 69.85) (end 111.83 69.595) (width 1) (layer "F.Cu") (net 13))
 (segment (start 104.845 78.105) (end 104.845 83.185) (width 1) (layer "F.Cu") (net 13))
 (segment (start 113.735 68.96) (end 112.845 68.96) (width 1) (layer "F.Cu") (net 13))
 (segment (start 111.83 69.85) (end 111.83 71.12) (width 1) (layer "F.Cu") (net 13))
 (segment (start 123.005 68.96) (end 113.735 68.96) (width 1) (layer "F.Cu") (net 13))
 (segment (start 113.735 68.96) (end 112.72 68.96) (width 1) (layer "F.Cu") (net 13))
 (segment (start 111.83 71.12) (end 109.29 73.66) (width 1) (layer "F.Cu") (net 13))
 (segment (start 111.83 57.15) (end 111.83 67.945) (width 1) (layer "F.Cu") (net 13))
 (segment (start 109.29 73.66) (end 104.845 78.105) (width 1) (layer "F.Cu") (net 13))
 (segment (start 113.735 68.96) (end 113.1 68.96) (width 1) (layer "F.Cu") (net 13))
 (segment (start 112.465 68.96) (end 112.465 68.58) (width 1) (layer "F.Cu") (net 13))
 (segment (start 124.276 68.96) (end 122.45 68.96) (width 1) (layer "F.Cu") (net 13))
 (segment (start 113.1 68.96) (end 112.465 68.96) (width 1) (layer "F.Cu") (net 13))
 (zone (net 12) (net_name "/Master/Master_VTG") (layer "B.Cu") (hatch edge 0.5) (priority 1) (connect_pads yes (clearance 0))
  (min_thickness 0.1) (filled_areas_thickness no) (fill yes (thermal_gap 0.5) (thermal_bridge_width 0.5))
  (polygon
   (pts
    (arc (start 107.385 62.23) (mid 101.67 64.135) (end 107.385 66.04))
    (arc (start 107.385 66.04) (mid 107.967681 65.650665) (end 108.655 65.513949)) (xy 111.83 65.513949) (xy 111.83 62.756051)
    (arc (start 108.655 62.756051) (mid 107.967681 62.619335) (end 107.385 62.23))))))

